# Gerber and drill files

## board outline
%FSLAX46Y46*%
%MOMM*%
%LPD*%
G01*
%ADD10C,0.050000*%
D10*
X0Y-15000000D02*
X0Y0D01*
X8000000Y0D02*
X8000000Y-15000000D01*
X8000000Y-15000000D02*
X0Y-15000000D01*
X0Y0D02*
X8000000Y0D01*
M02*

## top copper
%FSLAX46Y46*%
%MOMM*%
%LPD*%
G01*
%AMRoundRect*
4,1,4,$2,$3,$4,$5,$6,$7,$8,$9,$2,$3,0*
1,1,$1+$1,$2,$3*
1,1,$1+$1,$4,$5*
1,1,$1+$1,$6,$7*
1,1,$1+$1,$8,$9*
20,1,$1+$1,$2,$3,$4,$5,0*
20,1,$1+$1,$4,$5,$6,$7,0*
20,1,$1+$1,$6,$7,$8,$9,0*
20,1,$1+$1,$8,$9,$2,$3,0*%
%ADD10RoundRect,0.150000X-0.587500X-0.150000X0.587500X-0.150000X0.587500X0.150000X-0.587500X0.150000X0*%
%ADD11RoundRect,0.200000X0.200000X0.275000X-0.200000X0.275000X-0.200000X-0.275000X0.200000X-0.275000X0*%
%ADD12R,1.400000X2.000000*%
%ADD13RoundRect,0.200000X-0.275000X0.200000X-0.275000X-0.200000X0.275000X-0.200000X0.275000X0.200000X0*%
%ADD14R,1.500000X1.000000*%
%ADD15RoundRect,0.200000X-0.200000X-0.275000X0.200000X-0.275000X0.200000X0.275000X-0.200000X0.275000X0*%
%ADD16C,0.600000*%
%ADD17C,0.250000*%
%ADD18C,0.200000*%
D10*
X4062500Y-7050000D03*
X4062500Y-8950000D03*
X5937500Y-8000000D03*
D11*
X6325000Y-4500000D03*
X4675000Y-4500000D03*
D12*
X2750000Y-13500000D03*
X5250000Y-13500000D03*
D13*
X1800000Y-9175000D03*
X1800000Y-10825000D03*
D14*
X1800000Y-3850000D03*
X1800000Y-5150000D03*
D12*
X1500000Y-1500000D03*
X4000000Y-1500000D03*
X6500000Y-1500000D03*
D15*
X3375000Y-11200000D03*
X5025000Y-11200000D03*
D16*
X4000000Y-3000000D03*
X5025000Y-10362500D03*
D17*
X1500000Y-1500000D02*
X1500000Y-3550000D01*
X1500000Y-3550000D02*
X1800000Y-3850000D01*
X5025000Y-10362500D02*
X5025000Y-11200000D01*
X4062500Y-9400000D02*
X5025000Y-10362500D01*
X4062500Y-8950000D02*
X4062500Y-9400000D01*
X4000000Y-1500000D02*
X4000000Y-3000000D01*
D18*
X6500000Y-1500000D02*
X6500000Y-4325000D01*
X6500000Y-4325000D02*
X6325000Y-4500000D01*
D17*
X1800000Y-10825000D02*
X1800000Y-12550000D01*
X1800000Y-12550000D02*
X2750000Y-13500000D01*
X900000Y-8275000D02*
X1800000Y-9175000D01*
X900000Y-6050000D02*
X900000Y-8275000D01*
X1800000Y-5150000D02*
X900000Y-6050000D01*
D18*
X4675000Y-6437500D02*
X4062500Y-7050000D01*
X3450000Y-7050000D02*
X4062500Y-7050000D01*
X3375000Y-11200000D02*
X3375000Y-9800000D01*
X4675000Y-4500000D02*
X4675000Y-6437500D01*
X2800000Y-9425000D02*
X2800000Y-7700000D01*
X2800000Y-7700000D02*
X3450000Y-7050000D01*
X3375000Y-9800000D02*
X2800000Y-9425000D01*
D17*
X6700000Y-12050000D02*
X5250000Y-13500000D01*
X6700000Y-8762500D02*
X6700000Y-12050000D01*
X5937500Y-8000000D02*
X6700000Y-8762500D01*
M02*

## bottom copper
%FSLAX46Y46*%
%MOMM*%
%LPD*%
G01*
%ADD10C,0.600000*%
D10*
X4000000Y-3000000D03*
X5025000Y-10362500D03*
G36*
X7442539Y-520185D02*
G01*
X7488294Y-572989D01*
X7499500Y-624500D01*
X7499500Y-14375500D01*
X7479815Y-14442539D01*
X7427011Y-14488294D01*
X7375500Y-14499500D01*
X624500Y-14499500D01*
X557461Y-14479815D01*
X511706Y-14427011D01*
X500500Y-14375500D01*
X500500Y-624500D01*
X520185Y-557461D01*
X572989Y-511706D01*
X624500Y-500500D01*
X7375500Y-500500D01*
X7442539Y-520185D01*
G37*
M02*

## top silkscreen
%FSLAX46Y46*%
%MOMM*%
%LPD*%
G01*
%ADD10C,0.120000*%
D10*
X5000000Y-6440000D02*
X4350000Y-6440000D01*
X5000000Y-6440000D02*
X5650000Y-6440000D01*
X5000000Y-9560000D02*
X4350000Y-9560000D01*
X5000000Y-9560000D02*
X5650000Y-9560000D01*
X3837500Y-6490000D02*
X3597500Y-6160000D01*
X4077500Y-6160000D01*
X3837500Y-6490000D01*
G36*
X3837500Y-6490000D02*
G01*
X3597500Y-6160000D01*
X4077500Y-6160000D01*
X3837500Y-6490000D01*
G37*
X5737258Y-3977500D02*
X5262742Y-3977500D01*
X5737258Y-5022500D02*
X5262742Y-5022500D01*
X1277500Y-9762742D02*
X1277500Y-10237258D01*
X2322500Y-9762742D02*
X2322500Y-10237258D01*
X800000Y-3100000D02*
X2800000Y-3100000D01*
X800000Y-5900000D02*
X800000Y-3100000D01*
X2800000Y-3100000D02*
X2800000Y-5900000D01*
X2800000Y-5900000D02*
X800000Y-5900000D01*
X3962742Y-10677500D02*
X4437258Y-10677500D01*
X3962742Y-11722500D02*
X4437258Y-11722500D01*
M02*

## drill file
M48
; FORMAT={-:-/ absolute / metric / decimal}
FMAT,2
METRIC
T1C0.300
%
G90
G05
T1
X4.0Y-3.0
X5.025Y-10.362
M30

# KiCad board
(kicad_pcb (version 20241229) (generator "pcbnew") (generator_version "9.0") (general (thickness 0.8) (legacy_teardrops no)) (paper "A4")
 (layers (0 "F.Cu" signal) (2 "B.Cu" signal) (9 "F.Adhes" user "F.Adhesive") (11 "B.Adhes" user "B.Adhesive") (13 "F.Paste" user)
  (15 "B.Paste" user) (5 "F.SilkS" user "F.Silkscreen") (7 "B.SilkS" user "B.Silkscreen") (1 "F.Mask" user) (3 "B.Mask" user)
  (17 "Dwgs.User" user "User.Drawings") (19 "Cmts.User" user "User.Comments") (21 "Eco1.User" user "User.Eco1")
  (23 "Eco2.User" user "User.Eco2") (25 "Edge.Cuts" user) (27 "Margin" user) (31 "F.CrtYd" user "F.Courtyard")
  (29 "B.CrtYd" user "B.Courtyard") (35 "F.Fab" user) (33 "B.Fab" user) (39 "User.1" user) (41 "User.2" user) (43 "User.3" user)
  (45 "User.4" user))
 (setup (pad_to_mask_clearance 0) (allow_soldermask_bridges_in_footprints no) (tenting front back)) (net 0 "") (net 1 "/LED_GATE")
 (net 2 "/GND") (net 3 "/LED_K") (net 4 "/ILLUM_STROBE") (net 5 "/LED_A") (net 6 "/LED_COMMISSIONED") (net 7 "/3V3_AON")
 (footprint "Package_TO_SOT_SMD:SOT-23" (layer "F.Cu") (at 5 8)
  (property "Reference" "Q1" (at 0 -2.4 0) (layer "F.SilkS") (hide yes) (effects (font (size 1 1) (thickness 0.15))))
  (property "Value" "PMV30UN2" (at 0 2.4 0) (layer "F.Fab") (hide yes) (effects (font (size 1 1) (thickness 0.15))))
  (fp_line (start 0 -1.56) (end -0.65 -1.56) (stroke (width 0.12) (type solid)) (layer "F.SilkS"))
  (fp_line (start 0 -1.56) (end 0.65 -1.56) (stroke (width 0.12) (type solid)) (layer "F.SilkS"))
  (fp_line (start 0 1.56) (end -0.65 1.56) (stroke (width 0.12) (type solid)) (layer "F.SilkS"))
  (fp_line (start 0 1.56) (end 0.65 1.56) (stroke (width 0.12) (type solid)) (layer "F.SilkS"))
  (fp_poly (pts (xy -1.1625 -1.51) (xy -1.4025 -1.84) (xy -0.9225 -1.84)) (stroke (width 0.12) (type solid)) (fill yes) (layer "F.SilkS"))
  (pad "1" smd roundrect (at -0.9375 -0.95) (size 1.475 0.6) (layers "F.Cu" "F.Mask" "F.Paste") (roundrect_rratio 0.25) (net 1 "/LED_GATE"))
  (pad "2" smd roundrect (at -0.9375 0.95) (size 1.475 0.6) (layers "F.Cu" "F.Mask" "F.Paste") (roundrect_rratio 0.25) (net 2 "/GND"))
  (pad "3" smd roundrect (at 0.9375 0) (size 1.475 0.6) (layers "F.Cu" "F.Mask" "F.Paste") (roundrect_rratio 0.25) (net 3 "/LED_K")))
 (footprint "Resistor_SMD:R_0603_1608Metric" (layer "F.Cu") (at 5.5 4.5 180)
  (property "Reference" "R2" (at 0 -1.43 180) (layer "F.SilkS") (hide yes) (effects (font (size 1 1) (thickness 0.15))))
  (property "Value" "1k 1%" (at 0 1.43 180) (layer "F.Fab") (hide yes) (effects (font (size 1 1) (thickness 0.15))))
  (fp_line (start -0.237258 0.5225) (end 0.237258 0.5225) (stroke (width 0.12) (type solid)) (layer "F.SilkS"))
  (fp_line (start -0.237258 -0.5225) (end 0.237258 -0.5225) (stroke (width 0.12) (type solid)) (layer "F.SilkS"))
  (pad "1" smd roundrect (at -0.825 0 180) (size 0.8 0.95) (layers "F.Cu" "F.Mask" "F.Paste") (roundrect_rratio 0.25)
   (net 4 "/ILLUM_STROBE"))
  (pad "2" smd roundrect (at 0.825 0 180) (size 0.8 0.95) (layers "F.Cu" "F.Mask" "F.Paste") (roundrect_rratio 0.25) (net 1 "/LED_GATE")))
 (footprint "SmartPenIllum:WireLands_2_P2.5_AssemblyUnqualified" (layer "F.Cu") (at 4 13.5)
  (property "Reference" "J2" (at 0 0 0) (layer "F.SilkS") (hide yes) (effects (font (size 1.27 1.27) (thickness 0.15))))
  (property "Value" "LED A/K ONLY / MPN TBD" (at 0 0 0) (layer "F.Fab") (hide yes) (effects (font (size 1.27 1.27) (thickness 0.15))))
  (pad "1" smd rect (at -1.25 0) (size 1.4 2) (layers "F.Cu" "F.Mask") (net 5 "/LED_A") (thermal_bridge_angle 45))
  (pad "2" smd rect (at 1.25 0) (size 1.4 2) (layers "F.Cu" "F.Mask") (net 3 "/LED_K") (thermal_bridge_angle 45)))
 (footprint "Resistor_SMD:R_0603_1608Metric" (layer "F.Cu") (at 1.8 10 -90)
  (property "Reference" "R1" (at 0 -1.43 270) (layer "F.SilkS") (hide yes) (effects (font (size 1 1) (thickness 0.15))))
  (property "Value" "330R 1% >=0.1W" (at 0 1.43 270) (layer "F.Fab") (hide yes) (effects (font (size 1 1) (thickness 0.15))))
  (fp_line (start -0.237258 0.5225) (end 0.237258 0.5225) (stroke (width 0.12) (type solid)) (layer "F.SilkS"))
  (fp_line (start -0.237258 -0.5225) (end 0.237258 -0.5225) (stroke (width 0.12) (type solid)) (layer "F.SilkS"))
  (pad "1" smd roundrect (at -0.825 0 270) (size 0.8 0.95) (layers "F.Cu" "F.Mask" "F.Paste") (roundrect_rratio 0.25)
   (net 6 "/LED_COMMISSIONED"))
  (pad "2" smd roundrect (at 0.825 0 270) (size 0.8 0.95) (layers "F.Cu" "F.Mask" "F.Paste") (roundrect_rratio 0.25) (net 5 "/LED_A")))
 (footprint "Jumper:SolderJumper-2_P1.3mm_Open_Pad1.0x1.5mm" (layer "F.Cu") (at 1.8 4.5 -90)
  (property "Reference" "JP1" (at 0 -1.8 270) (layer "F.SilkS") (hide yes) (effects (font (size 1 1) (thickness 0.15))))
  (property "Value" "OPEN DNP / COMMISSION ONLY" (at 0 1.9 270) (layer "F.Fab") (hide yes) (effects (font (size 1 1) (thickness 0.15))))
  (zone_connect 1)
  (fp_line (start -1.4 1) (end -1.4 -1) (stroke (width 0.12) (type solid)) (layer "F.SilkS"))
  (fp_line (start 1.4 1) (end -1.4 1) (stroke (width 0.12) (type solid)) (layer "F.SilkS"))
  (fp_line (start -1.4 -1) (end 1.4 -1) (stroke (width 0.12) (type solid)) (layer "F.SilkS"))
  (fp_line (start 1.4 -1) (end 1.4 1) (stroke (width 0.12) (type solid)) (layer "F.SilkS"))
  (pad "1" smd rect (at -0.65 0 270) (size 1 1.5) (layers "F.Cu" "F.Mask") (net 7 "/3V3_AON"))
  (pad "2" smd rect (at 0.65 0 270) (size 1 1.5) (layers "F.Cu" "F.Mask") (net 6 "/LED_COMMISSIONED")))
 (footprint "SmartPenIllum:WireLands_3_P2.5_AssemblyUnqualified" (layer "F.Cu") (at 4 1.5)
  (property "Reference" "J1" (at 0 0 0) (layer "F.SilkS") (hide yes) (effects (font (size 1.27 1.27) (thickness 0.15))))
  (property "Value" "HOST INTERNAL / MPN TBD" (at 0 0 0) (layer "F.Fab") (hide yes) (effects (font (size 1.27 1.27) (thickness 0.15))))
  (pad "1" smd rect (at -2.5 0) (size 1.4 2) (layers "F.Cu" "F.Mask") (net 7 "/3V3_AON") (thermal_bridge_angle 45))
  (pad "2" smd rect (at 0 0) (size 1.4 2) (layers "F.Cu" "F.Mask") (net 2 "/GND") (thermal_bridge_angle 45))
  (pad "3" smd rect (at 2.5 0) (size 1.4 2) (layers "F.Cu" "F.Mask") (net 4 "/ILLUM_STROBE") (thermal_bridge_angle 45)))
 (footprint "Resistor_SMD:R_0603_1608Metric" (layer "F.Cu") (at 4.2 11.2)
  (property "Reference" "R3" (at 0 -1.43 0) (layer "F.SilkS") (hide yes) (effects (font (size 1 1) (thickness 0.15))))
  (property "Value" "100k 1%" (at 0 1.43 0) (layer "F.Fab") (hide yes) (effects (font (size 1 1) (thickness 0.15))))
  (fp_line (start -0.237258 -0.5225) (end 0.237258 -0.5225) (stroke (width 0.12) (type solid)) (layer "F.SilkS"))
  (fp_line (start -0.237258 0.5225) (end 0.237258 0.5225) (stroke (width 0.12) (type solid)) (layer "F.SilkS"))
  (pad "1" smd roundrect (at -0.825 0) (size 0.8 0.95) (layers "F.Cu" "F.Mask" "F.Paste") (roundrect_rratio 0.25) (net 1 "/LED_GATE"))
  (pad "2" smd roundrect (at 0.825 0) (size 0.8 0.95) (layers "F.Cu" "F.Mask" "F.Paste") (roundrect_rratio 0.25) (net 2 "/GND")))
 (gr_line (start 0 15) (end 0 0) (stroke (width 0.05) (type default)) (layer "Edge.Cuts"))
 (gr_line (start 8 0) (end 8 15) (stroke (width 0.05) (type default)) (layer "Edge.Cuts"))
 (gr_line (start 8 15) (end 0 15) (stroke (width 0.05) (type default)) (layer "Edge.Cuts"))
 (gr_line (start 0 0) (end 8 0) (stroke (width 0.05) (type default)) (layer "Edge.Cuts"))
 (segment (start 1.5 1.5) (end 1.5 3.55) (width 0.25) (layer "F.Cu") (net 7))
 (segment (start 1.5 3.55) (end 1.8 3.85) (width 0.25) (layer "F.Cu") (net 7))
 (segment (start 5.025 10.3625) (end 5.025 11.2) (width 0.25) (layer "F.Cu") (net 2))
 (segment (start 4.0625 9.4) (end 5.025 10.3625) (width 0.25) (layer "F.Cu") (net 2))
 (segment (start 4.0625 8.95) (end 4.0625 9.4) (width 0.25) (layer "F.Cu") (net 2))
 (segment (start 4 1.5) (end 4 3) (width 0.25) (layer "F.Cu") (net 2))
 (via (at 4 3) (size 0.6) (drill 0.3) (layers "F.Cu" "B.Cu") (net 2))
 (via (at 5.025 10.3625) (size 0.6) (drill 0.3) (layers "F.Cu" "B.Cu") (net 2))
 (segment (start 6.5 1.5) (end 6.5 4.325) (width 0.2) (layer "F.Cu") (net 4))
 (segment (start 6.5 4.325) (end 6.325 4.5) (width 0.2) (layer "F.Cu") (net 4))
 (segment (start 1.8 10.825) (end 1.8 12.55) (width 0.25) (layer "F.Cu") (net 5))
 (segment (start 1.8 12.55) (end 2.75 13.5) (width 0.25) (layer "F.Cu") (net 5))
 (segment (start 0.9 8.275) (end 1.8 9.175) (width 0.25) (layer "F.Cu") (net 6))
 (segment (start 0.9 6.05) (end 0.9 8.275) (width 0.25) (layer "F.Cu") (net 6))
 (segment (start 1.8 5.15) (end 0.9 6.05) (width 0.25) (layer "F.Cu") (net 6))
 (segment (start 4.675 6.4375) (end 4.0625 7.05) (width 0.2) (layer "F.Cu") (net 1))
 (segment (start 3.45 7.05) (end 4.0625 7.05) (width 0.2) (layer "F.Cu") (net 1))
 (segment (start 3.375 11.2) (end 3.375 9.8) (width 0.2) (layer "F.Cu") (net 1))
 (segment (start 4.675 4.5) (end 4.675 6.4375) (width 0.2) (layer "F.Cu") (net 1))
 (segment (start 2.8 9.425) (end 2.8 7.7) (width 0.2) (layer "F.Cu") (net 1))
 (segment (start 2.8 7.7) (end 3.45 7.05) (width 0.2) (layer "F.Cu") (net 1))
 (segment (start 3.375 9.8) (end 2.8 9.425) (width 0.2) (layer "F.Cu") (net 1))
 (segment (start 6.7 12.05) (end 5.25 13.5) (width 0.25) (layer "F.Cu") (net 3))
 (segment (start 6.7 8.7625) (end 6.7 12.05) (width 0.25) (layer "F.Cu") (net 3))
 (segment (start 5.9375 8) (end 6.7 8.7625) (width 0.25) (layer "F.Cu") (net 3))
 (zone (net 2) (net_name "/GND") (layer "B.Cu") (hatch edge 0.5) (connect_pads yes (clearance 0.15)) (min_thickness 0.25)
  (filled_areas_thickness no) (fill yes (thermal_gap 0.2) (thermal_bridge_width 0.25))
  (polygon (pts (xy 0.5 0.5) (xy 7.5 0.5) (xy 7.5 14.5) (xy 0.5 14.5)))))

